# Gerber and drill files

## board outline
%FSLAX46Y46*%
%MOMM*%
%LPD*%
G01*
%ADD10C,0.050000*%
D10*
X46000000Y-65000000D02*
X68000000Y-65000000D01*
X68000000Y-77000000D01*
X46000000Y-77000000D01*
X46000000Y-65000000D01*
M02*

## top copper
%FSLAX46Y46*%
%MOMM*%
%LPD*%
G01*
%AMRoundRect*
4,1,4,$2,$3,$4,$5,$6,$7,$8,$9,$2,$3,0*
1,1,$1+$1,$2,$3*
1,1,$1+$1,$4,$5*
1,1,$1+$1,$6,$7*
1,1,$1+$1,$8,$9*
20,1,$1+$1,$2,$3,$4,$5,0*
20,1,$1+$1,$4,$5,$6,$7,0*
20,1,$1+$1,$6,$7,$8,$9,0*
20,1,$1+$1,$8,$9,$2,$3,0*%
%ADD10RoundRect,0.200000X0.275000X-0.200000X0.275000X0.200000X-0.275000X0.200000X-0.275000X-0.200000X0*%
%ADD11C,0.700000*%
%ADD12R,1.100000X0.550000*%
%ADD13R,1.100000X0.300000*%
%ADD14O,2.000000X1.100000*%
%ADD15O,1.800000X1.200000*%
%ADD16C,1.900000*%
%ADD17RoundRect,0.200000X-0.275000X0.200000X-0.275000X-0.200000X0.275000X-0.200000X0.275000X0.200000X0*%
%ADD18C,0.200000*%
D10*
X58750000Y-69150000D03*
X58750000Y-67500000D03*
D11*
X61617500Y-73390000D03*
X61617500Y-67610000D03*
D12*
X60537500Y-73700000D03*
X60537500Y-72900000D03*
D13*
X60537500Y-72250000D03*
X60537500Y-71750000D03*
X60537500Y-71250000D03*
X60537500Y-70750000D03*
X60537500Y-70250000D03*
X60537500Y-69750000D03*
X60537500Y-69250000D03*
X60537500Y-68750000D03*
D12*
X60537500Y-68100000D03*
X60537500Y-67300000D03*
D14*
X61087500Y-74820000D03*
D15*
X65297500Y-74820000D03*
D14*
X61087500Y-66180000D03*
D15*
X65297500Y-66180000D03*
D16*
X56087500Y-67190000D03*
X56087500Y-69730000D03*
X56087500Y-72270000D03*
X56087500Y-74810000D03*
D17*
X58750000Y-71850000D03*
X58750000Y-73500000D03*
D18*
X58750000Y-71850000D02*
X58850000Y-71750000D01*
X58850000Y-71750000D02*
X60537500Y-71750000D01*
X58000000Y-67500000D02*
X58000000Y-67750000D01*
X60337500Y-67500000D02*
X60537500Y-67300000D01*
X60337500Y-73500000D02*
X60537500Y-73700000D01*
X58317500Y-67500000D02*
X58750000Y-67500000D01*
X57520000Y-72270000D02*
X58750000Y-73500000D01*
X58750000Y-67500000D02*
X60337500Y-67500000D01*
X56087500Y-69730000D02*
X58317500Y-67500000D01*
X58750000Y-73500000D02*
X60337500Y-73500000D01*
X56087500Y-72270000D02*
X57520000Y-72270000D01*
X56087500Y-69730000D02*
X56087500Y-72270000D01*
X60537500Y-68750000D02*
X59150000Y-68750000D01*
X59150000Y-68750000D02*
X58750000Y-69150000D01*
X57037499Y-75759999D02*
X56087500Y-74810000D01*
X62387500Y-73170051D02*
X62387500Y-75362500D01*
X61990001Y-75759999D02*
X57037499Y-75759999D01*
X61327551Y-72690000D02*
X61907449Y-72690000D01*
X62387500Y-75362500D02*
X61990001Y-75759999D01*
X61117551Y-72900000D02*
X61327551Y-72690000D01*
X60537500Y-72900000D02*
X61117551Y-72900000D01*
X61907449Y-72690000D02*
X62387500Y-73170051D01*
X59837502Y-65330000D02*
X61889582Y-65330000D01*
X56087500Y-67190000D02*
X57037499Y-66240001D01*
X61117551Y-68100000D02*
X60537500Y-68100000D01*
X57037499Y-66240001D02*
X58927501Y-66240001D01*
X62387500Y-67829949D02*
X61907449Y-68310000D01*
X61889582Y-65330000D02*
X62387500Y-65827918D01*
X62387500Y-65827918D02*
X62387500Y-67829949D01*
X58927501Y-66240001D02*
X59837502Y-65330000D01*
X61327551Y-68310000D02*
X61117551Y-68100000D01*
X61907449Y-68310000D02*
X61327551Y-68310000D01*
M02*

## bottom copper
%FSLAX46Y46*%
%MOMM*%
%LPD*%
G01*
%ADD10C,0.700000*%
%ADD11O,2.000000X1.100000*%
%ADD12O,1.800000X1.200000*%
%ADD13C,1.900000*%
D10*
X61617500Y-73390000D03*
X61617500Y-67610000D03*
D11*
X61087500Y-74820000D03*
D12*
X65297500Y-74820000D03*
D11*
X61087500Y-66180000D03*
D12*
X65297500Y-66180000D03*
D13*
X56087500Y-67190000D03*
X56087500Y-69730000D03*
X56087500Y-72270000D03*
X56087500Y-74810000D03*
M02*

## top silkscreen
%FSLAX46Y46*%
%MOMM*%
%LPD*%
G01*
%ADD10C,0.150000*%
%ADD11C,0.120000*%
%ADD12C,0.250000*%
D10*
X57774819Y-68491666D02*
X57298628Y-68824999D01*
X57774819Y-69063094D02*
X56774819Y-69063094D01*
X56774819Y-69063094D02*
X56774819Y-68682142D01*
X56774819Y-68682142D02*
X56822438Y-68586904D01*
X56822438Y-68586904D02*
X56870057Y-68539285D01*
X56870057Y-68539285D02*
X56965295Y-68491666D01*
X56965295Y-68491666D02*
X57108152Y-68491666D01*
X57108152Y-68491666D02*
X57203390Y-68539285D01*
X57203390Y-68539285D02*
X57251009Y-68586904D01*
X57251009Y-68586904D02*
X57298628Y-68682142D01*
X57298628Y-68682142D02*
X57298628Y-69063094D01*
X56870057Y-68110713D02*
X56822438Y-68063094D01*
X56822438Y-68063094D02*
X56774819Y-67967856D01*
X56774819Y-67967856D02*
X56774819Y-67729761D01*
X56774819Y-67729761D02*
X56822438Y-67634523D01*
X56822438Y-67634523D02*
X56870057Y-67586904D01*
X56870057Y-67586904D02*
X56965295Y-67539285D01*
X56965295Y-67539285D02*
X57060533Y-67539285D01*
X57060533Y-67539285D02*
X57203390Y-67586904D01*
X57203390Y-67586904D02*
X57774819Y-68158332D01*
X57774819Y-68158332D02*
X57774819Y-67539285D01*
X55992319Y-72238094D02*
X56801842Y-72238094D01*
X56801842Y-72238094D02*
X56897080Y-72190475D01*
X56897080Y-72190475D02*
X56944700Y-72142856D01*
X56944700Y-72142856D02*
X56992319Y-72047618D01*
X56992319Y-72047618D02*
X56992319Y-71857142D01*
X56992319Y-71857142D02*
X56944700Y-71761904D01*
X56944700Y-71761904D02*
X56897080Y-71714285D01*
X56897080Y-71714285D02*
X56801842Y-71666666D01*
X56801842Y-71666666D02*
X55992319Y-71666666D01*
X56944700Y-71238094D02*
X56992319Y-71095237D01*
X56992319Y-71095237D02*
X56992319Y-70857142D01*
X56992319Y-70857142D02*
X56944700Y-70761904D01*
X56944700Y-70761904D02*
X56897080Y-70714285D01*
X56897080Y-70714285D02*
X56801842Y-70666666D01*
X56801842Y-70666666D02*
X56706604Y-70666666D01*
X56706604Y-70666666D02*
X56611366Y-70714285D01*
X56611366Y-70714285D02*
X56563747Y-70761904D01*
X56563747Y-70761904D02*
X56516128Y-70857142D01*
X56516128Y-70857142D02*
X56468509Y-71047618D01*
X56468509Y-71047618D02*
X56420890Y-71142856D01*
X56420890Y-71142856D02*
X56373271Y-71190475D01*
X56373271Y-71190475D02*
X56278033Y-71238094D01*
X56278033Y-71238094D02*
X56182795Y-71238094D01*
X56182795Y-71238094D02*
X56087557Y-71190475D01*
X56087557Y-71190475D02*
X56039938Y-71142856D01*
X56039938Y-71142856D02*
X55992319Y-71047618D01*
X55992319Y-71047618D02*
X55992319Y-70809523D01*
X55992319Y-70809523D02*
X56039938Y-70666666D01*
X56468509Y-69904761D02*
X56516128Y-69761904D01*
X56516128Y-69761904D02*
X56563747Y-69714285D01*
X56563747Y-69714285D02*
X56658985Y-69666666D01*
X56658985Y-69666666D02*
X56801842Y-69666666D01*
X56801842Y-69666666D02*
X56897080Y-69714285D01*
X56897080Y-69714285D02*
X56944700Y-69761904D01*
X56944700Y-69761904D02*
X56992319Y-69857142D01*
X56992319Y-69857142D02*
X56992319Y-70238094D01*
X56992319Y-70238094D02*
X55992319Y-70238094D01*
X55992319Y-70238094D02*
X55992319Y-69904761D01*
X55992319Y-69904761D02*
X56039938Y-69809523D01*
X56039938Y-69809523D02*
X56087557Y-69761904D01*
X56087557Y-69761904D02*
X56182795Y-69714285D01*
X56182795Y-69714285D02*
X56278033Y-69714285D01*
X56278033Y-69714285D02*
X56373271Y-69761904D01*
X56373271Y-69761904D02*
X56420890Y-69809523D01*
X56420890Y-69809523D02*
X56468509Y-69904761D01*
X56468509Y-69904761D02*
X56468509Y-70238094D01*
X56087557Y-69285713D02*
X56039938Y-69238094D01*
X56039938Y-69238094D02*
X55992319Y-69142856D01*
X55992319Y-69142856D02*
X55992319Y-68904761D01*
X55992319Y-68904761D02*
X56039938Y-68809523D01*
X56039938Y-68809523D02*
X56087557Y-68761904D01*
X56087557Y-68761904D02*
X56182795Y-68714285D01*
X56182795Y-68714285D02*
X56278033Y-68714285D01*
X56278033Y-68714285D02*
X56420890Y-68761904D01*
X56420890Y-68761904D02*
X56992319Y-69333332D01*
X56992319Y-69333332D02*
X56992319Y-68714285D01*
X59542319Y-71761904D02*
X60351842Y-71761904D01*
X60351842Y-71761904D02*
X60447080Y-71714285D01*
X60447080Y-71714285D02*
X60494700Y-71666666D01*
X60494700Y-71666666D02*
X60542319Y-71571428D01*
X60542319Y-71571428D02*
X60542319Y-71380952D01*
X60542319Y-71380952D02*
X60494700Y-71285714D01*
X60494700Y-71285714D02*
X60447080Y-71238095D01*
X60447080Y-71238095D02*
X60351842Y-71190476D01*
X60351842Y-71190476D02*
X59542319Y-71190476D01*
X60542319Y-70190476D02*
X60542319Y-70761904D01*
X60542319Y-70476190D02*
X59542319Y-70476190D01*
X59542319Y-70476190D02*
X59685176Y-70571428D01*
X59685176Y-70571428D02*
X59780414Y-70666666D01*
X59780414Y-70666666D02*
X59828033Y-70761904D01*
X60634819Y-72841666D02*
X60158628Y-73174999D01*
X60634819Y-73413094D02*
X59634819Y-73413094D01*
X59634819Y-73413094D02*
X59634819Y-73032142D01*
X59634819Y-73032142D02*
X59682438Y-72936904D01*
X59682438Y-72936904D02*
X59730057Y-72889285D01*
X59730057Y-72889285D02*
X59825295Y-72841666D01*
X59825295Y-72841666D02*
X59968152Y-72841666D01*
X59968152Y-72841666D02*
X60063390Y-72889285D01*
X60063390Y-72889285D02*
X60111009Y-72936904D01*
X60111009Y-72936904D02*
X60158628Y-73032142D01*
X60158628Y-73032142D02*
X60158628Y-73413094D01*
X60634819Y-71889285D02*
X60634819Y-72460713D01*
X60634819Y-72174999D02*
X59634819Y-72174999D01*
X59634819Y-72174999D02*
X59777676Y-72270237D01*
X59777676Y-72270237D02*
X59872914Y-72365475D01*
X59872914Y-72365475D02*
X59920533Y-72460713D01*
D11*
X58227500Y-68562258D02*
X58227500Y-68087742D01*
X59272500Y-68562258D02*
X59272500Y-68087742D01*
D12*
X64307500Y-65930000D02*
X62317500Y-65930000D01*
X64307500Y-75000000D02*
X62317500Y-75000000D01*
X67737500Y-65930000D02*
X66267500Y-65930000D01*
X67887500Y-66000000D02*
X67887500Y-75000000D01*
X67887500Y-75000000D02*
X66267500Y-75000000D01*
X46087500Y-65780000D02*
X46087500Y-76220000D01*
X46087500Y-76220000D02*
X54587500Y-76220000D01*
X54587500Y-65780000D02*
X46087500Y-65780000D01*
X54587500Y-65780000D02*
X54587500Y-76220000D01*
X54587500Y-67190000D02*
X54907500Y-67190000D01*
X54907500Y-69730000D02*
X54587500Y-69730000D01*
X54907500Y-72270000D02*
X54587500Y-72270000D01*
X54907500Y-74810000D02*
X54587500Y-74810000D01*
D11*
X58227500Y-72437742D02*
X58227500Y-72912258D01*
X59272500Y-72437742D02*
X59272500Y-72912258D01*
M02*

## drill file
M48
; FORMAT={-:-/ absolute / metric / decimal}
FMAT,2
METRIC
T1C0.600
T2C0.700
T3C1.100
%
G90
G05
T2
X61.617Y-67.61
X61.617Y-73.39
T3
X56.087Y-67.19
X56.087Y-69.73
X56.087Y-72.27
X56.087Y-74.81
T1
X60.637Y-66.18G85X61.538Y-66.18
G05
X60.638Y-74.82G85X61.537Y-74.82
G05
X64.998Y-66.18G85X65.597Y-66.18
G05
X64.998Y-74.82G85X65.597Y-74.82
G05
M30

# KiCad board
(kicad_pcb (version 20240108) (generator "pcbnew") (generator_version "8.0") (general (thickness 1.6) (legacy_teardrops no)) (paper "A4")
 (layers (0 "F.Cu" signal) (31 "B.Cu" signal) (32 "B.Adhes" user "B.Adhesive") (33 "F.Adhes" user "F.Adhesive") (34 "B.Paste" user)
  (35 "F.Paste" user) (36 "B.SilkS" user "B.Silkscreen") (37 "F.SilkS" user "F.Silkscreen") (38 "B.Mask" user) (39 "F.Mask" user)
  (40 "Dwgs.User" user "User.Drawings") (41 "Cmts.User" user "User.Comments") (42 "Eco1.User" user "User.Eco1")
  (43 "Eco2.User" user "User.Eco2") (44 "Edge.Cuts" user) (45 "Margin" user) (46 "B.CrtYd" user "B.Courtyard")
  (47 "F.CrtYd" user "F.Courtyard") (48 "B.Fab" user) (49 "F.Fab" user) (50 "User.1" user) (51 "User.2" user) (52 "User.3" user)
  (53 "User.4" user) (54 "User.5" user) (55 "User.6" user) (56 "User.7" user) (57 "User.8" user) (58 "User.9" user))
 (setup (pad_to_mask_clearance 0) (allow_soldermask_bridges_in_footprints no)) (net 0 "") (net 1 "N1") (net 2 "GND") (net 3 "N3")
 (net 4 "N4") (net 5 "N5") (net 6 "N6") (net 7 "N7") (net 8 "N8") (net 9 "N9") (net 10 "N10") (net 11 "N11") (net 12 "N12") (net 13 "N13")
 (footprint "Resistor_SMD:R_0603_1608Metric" (layer "F.Cu") (at 58.75 68.325 90)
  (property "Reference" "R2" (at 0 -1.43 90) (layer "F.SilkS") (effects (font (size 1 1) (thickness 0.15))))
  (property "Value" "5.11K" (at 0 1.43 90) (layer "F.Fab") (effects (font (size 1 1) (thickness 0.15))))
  (fp_line (start -0.237258 -0.5225) (end 0.237258 -0.5225) (stroke (width 0.12) (type solid)) (layer "F.SilkS"))
  (fp_line (start -0.237258 0.5225) (end 0.237258 0.5225) (stroke (width 0.12) (type solid)) (layer "F.SilkS"))
  (pad "1" smd roundrect (at -0.825 0 90) (size 0.8 0.95) (layers "F.Cu" "F.Paste" "F.Mask") (roundrect_rratio 0.25) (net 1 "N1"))
  (pad "2" smd roundrect (at 0.825 0 90) (size 0.8 0.95) (layers "F.Cu" "F.Paste" "F.Mask") (roundrect_rratio 0.25) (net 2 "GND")))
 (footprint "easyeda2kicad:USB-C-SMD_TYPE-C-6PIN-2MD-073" (layer "F.Cu") (at 62.9175 70.5 90)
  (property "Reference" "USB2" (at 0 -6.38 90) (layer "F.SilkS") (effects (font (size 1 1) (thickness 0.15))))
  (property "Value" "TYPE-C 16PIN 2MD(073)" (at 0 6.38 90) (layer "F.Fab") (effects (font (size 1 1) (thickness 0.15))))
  (fp_line (start 4.57 1.39) (end 4.57 -0.6) (stroke (width 0.25) (type solid)) (layer "F.SilkS"))
  (fp_line (start -4.5 1.39) (end -4.5 -0.6) (stroke (width 0.25) (type solid)) (layer "F.SilkS"))
  (fp_line (start 4.57 4.82) (end 4.57 3.35) (stroke (width 0.25) (type solid)) (layer "F.SilkS"))
  (fp_line (start 4.5 4.97) (end -4.5 4.97) (stroke (width 0.25) (type solid)) (layer "F.SilkS"))
  (fp_line (start -4.5 4.97) (end -4.5 3.35) (stroke (width 0.25) (type solid)) (layer "F.SilkS"))
  (pad "" thru_hole circle (at -2.89 -1.3 90) (size 0.7 0.7) (drill 0.7) (layers "*.Cu" "*.Mask") (remove_unused_layers no))
  (pad "" thru_hole circle (at 2.89 -1.3 90) (size 0.7 0.7) (drill 0.7) (layers "*.Cu" "*.Mask") (remove_unused_layers no))
  (pad "1" smd rect (at -3.2 -2.38 90) (size 0.55 1.1) (layers "F.Cu" "F.Paste" "F.Mask") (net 2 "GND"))
  (pad "2" smd rect (at -2.4 -2.38 90) (size 0.55 1.1) (layers "F.Cu" "F.Paste" "F.Mask") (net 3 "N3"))
  (pad "3" smd rect (at -1.75 -2.38 90) (size 0.3 1.1) (layers "F.Cu" "F.Paste" "F.Mask") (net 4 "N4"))
  (pad "4" smd rect (at -1.25 -2.38 90) (size 0.3 1.1) (layers "F.Cu" "F.Paste" "F.Mask") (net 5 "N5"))
  (pad "5" smd rect (at -0.75 -2.38 90) (size 0.3 1.1) (layers "F.Cu" "F.Paste" "F.Mask") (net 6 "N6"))
  (pad "6" smd rect (at -0.25 -2.38 90) (size 0.3 1.1) (layers "F.Cu" "F.Paste" "F.Mask") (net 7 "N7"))
  (pad "7" smd rect (at 0.25 -2.38 90) (size 0.3 1.1) (layers "F.Cu" "F.Paste" "F.Mask") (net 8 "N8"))
  (pad "8" smd rect (at 0.75 -2.38 90) (size 0.3 1.1) (layers "F.Cu" "F.Paste" "F.Mask") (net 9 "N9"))
  (pad "9" smd rect (at 1.25 -2.38 90) (size 0.3 1.1) (layers "F.Cu" "F.Paste" "F.Mask") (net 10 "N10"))
  (pad "10" smd rect (at 1.75 -2.38 90) (size 0.3 1.1) (layers "F.Cu" "F.Paste" "F.Mask") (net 1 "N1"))
  (pad "11" smd rect (at 2.4 -2.38 90) (size 0.55 1.1) (layers "F.Cu" "F.Paste" "F.Mask") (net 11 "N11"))
  (pad "12" smd rect (at 3.2 -2.38 90) (size 0.55 1.1) (layers "F.Cu" "F.Paste" "F.Mask") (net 2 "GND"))
  (pad "13" thru_hole oval (at -4.32 -1.83 90) (size 1.1 2) (drill oval 0.599999 1.499997) (layers "*.Cu" "*.Mask")
   (remove_unused_layers no) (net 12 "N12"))
  (pad "13" thru_hole oval (at -4.32 2.38 90) (size 1.2 1.8) (drill oval 0.599999 1.199998) (layers "*.Cu" "*.Mask")
   (remove_unused_layers no) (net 12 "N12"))
  (pad "14" thru_hole oval (at 4.32 -1.83 90) (size 1.1 2) (drill oval 0.599999 1.500022) (layers "*.Cu" "*.Mask") (remove_unused_layers no)
   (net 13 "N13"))
  (pad "14" thru_hole oval (at 4.32 2.38 90) (size 1.2 1.8) (drill oval 0.599999 1.199998) (layers "*.Cu" "*.Mask")
   (remove_unused_layers no) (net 13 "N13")))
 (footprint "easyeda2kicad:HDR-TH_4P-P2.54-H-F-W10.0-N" (layer "F.Cu") (at 56.0875 71 -90)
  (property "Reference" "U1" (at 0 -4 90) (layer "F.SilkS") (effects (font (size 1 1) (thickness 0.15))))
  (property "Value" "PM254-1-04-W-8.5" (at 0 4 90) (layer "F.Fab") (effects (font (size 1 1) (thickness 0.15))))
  (fp_line (start -5.22 10) (end 5.22 10) (stroke (width 0.25) (type solid)) (layer "F.SilkS"))
  (fp_line (start 5.22 10) (end 5.22 1.5) (stroke (width 0.25) (type solid)) (layer "F.SilkS"))
  (fp_line (start -5.22 1.5) (end -5.22 10) (stroke (width 0.25) (type solid)) (layer "F.SilkS"))
  (fp_line (start -5.22 1.5) (end 5.22 1.5) (stroke (width 0.25) (type solid)) (layer "F.SilkS"))
  (fp_line (start -3.81 1.5) (end -3.81 1.18) (stroke (width 0.25) (type solid)) (layer "F.SilkS"))
  (fp_line (start -1.27 1.18) (end -1.27 1.5) (stroke (width 0.25) (type solid)) (layer "F.SilkS"))
  (fp_line (start 1.27 1.18) (end 1.27 1.5) (stroke (width 0.25) (type solid)) (layer "F.SilkS"))
  (fp_line (start 3.81 1.18) (end 3.81 1.5) (stroke (width 0.25) (type solid)) (layer "F.SilkS"))
  (pad "1" thru_hole circle (at -3.81 0 270) (size 1.9 1.9) (drill 1.100023) (layers "*.Cu" "*.Mask") (remove_unused_layers no)
   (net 11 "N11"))
  (pad "2" thru_hole circle (at -1.27 0 270) (size 1.9 1.9) (drill 1.100023) (layers "*.Cu" "*.Mask") (remove_unused_layers no)
   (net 2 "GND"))
  (pad "3" thru_hole circle (at 1.27 0 270) (size 1.9 1.9) (drill 1.100023) (layers "*.Cu" "*.Mask") (remove_unused_layers no) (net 2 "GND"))
  (pad "4" thru_hole circle (at 3.81 0 270) (size 1.9 1.9) (drill 1.100023) (layers "*.Cu" "*.Mask") (remove_unused_layers no) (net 3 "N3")))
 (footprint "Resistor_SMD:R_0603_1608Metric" (layer "F.Cu") (at 58.75 72.675 -90)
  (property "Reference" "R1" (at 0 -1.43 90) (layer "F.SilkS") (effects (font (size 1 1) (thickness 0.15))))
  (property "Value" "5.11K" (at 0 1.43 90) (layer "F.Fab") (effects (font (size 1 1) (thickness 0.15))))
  (fp_line (start -0.237258 0.5225) (end 0.237258 0.5225) (stroke (width 0.12) (type solid)) (layer "F.SilkS"))
  (fp_line (start -0.237258 -0.5225) (end 0.237258 -0.5225) (stroke (width 0.12) (type solid)) (layer "F.SilkS"))
  (pad "1" smd roundrect (at -0.825 0 270) (size 0.8 0.95) (layers "F.Cu" "F.Paste" "F.Mask") (roundrect_rratio 0.25) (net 5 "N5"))
  (pad "2" smd roundrect (at 0.825 0 270) (size 0.8 0.95) (layers "F.Cu" "F.Paste" "F.Mask") (roundrect_rratio 0.25) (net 2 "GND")))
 (gr_rect (start 46 65) (end 68 77) (stroke (width 0.05) (type default)) (fill none) (layer "Edge.Cuts"))
 (segment (start 58.75 71.85) (end 58.85 71.75) (width 0.2) (layer "F.Cu") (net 5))
 (segment (start 58.85 71.75) (end 60.5375 71.75) (width 0.2) (layer "F.Cu") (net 5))
 (segment (start 58 67.5) (end 58 67.75) (width 0.2) (layer "F.Cu") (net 2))
 (segment (start 60.3375 67.5) (end 60.5375 67.3) (width 0.2) (layer "F.Cu") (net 2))
 (segment (start 60.3375 73.5) (end 60.5375 73.7) (width 0.2) (layer "F.Cu") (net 2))
 (segment (start 58.3175 67.5) (end 58.75 67.5) (width 0.2) (layer "F.Cu") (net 2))
 (segment (start 57.52 72.27) (end 58.75 73.5) (width 0.2) (layer "F.Cu") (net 2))
 (segment (start 58.75 67.5) (end 60.3375 67.5) (width 0.2) (layer "F.Cu") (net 2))
 (segment (start 56.0875 69.73) (end 58.3175 67.5) (width 0.2) (layer "F.Cu") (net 2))
 (segment (start 58.75 73.5) (end 60.3375 73.5) (width 0.2) (layer "F.Cu") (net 2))
 (segment (start 56.0875 72.27) (end 57.52 72.27) (width 0.2) (layer "F.Cu") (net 2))
 (segment (start 56.0875 69.73) (end 56.0875 72.27) (width 0.2) (layer "F.Cu") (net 2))
 (segment (start 60.5375 68.75) (end 59.15 68.75) (width 0.2) (layer "F.Cu") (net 1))
 (segment (start 59.15 68.75) (end 58.75 69.15) (width 0.2) (layer "F.Cu") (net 1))
 (segment (start 57.037499 75.759999) (end 56.0875 74.81) (width 0.2) (layer "F.Cu") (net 3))
 (segment (start 62.3875 73.170051) (end 62.3875 75.3625) (width 0.2) (layer "F.Cu") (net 3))
 (segment (start 61.990001 75.759999) (end 57.037499 75.759999) (width 0.2) (layer "F.Cu") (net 3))
 (segment (start 61.327551 72.69) (end 61.907449 72.69) (width 0.2) (layer "F.Cu") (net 3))
 (segment (start 62.3875 75.3625) (end 61.990001 75.759999) (width 0.2) (layer "F.Cu") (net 3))
 (segment (start 61.117551 72.9) (end 61.327551 72.69) (width 0.2) (layer "F.Cu") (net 3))
 (segment (start 60.5375 72.9) (end 61.117551 72.9) (width 0.2) (layer "F.Cu") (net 3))
 (segment (start 61.907449 72.69) (end 62.3875 73.170051) (width 0.2) (layer "F.Cu") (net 3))
 (segment (start 59.837502 65.33) (end 61.889582 65.33) (width 0.2) (layer "F.Cu") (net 11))
 (segment (start 56.0875 67.19) (end 57.037499 66.240001) (width 0.2) (layer "F.Cu") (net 11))
 (segment (start 61.117551 68.1) (end 60.5375 68.1) (width 0.2) (layer "F.Cu") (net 11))
 (segment (start 57.037499 66.240001) (end 58.927501 66.240001) (width 0.2) (layer "F.Cu") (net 11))
 (segment (start 62.3875 67.829949) (end 61.907449 68.31) (width 0.2) (layer "F.Cu") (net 11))
 (segment (start 61.889582 65.33) (end 62.3875 65.827918) (width 0.2) (layer "F.Cu") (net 11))
 (segment (start 62.3875 65.827918) (end 62.3875 67.829949) (width 0.2) (layer "F.Cu") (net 11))
 (segment (start 58.927501 66.240001) (end 59.837502 65.33) (width 0.2) (layer "F.Cu") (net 11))
 (segment (start 61.327551 68.31) (end 61.117551 68.1) (width 0.2) (layer "F.Cu") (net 11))
 (segment (start 61.907449 68.31) (end 61.327551 68.31) (width 0.2) (layer "F.Cu") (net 11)))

